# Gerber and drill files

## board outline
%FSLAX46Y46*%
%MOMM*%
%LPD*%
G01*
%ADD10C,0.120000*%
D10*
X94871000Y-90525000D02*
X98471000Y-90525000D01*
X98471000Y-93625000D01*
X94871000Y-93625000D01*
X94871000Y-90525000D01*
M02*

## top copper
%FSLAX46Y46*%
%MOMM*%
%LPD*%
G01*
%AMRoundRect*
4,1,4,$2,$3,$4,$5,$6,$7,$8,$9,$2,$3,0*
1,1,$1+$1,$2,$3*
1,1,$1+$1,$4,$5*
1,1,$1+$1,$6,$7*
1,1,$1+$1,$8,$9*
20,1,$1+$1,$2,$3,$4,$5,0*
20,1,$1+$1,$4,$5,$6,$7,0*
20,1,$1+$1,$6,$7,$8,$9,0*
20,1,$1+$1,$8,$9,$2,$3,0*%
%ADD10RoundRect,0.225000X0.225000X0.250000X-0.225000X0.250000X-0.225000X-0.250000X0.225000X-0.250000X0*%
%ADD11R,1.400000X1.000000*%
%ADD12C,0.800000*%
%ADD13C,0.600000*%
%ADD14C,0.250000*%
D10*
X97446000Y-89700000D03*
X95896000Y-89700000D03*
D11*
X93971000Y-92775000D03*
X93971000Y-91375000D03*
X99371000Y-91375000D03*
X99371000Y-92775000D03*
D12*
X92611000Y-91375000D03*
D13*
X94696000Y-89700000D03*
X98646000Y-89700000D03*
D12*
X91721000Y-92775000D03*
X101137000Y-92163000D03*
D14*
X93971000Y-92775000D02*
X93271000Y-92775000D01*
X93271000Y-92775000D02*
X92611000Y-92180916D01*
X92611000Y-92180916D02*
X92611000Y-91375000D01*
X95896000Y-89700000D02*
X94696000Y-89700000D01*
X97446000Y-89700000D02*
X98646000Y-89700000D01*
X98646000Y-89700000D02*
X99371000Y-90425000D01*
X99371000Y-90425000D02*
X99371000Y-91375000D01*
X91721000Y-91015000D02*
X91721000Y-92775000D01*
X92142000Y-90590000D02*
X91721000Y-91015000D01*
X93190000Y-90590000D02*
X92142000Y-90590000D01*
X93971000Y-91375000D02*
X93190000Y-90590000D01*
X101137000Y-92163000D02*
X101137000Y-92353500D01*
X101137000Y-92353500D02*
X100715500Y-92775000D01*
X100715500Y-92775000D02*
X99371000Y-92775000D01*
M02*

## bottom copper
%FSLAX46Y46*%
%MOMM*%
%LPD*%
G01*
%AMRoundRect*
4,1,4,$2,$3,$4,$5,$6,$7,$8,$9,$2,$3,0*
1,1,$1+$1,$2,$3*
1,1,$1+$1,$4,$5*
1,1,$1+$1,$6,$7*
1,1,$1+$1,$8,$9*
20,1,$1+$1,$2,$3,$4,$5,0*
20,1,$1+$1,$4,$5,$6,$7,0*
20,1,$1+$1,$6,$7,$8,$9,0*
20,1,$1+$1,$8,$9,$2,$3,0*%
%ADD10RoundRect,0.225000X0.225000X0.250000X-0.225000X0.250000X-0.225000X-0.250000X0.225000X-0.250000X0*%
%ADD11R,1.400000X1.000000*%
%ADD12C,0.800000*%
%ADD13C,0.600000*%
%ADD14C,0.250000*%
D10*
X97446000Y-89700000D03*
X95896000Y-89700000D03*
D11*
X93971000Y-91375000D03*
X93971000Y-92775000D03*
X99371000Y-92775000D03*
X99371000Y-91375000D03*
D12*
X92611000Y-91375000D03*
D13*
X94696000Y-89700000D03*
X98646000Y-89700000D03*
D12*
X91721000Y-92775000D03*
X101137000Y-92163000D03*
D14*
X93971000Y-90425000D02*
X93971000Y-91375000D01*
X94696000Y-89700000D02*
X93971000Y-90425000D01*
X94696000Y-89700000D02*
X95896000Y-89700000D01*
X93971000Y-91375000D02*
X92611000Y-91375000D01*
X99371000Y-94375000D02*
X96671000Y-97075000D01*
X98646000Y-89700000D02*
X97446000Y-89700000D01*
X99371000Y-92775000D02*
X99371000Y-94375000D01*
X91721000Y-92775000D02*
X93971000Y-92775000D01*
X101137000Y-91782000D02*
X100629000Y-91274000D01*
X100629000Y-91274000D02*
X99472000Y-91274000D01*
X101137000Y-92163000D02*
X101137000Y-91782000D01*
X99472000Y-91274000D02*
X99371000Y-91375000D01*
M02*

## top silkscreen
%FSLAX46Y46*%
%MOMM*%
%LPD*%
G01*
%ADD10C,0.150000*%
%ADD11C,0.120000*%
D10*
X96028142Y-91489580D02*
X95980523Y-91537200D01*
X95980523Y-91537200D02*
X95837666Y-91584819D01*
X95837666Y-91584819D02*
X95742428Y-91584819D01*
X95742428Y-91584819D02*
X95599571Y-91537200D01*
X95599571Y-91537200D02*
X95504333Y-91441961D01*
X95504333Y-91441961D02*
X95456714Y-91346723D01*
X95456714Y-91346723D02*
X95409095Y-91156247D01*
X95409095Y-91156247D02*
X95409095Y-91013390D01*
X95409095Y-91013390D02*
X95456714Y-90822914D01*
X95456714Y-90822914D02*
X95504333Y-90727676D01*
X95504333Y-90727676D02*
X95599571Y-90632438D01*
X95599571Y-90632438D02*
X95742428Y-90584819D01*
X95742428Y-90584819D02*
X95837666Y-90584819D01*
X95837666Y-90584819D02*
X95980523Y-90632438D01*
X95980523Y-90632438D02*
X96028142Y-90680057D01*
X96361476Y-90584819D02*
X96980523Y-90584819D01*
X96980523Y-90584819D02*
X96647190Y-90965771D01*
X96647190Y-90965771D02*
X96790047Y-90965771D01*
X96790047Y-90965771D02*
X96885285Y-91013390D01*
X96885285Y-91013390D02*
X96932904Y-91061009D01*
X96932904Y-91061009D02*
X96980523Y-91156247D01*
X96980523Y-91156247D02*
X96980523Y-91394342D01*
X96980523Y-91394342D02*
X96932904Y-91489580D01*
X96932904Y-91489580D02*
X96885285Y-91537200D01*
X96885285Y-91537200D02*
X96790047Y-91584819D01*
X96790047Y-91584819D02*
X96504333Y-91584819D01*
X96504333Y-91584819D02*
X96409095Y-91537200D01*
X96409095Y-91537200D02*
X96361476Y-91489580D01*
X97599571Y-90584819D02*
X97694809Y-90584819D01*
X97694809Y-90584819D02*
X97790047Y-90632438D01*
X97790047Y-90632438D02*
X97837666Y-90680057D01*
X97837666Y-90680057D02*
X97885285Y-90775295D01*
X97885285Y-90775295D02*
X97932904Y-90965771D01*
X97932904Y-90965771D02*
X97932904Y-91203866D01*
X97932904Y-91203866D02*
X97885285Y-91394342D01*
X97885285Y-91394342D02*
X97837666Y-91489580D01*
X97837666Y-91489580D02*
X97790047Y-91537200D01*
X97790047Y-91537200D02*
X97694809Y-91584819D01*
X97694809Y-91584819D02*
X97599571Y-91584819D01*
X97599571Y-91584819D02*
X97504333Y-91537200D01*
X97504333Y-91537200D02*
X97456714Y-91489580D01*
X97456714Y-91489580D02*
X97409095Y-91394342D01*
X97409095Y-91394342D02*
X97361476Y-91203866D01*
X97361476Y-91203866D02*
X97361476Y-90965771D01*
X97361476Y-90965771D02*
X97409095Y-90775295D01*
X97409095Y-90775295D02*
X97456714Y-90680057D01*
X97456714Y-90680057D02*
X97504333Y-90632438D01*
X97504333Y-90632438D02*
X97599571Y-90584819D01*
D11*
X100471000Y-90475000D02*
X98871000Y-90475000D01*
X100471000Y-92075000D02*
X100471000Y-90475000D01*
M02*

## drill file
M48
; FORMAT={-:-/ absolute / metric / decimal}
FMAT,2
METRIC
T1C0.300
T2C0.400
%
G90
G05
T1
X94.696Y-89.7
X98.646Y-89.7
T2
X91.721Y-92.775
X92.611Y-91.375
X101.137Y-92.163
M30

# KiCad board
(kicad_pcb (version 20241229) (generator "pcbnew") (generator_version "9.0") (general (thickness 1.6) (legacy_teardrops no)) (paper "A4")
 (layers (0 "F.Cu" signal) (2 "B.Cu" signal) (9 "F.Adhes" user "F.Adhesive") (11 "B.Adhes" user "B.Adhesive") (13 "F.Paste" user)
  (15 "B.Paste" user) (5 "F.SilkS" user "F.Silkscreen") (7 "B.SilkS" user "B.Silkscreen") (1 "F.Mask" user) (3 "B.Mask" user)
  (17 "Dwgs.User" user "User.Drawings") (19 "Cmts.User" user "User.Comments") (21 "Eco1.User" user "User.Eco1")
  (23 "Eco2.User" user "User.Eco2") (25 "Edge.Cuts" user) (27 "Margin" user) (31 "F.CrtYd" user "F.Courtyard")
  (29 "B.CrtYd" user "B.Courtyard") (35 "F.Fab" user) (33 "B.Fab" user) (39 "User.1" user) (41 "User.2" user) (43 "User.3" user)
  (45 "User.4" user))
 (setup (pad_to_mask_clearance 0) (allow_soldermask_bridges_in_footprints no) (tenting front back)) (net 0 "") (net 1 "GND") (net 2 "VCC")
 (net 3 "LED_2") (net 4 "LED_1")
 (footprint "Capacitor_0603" (layer "F.Cu") (at 96.671 89.7 180)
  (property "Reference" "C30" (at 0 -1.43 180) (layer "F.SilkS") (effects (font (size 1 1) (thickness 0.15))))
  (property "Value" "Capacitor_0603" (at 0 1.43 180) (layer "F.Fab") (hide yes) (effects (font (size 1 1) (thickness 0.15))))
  (pad "1" smd roundrect (at -0.775 0 180) (size 0.9 0.95) (layers "F.Cu" "F.Mask" "F.Paste") (roundrect_rratio 0.25) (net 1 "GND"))
  (pad "1" smd roundrect (at -0.775 0 180) (size 0.9 0.95) (layers "B.Cu" "B.Mask" "B.Paste") (roundrect_rratio 0.25) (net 1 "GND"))
  (pad "2" smd roundrect (at 0.775 0 180) (size 0.9 0.95) (layers "F.Cu" "F.Mask" "F.Paste") (roundrect_rratio 0.25) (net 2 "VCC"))
  (pad "2" smd roundrect (at 0.775 0 180) (size 0.9 0.95) (layers "B.Cu" "B.Mask" "B.Paste") (roundrect_rratio 0.25) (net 2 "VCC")))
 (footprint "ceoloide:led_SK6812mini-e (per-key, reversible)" (layer "B.Cu") (at 96.671 92.075 180)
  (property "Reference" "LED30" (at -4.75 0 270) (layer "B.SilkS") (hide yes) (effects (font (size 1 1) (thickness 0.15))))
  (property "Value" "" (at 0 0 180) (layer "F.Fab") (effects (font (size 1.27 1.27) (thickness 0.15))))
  (fp_line (start -3.8 1.6) (end -2.2 1.6) (stroke (width 0.12) (type solid)) (layer "F.SilkS"))
  (fp_line (start -3.8 0) (end -3.8 1.6) (stroke (width 0.12) (type solid)) (layer "F.SilkS"))
  (fp_rect (start -1.8 -1.55) (end 1.8 1.55) (stroke (width 0.12) (type solid)) (fill no) (layer "Edge.Cuts"))
  (pad "1" smd rect (at 2.7 -0.7 180) (size 1.4 1) (layers "F.Cu" "F.Mask" "F.Paste") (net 2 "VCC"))
  (pad "1" smd rect (at 2.7 0.7 180) (size 1.4 1) (layers "B.Cu" "B.Mask" "B.Paste") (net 2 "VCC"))
  (pad "2" smd rect (at 2.7 -0.7 180) (size 1.4 1) (layers "B.Cu" "B.Mask" "B.Paste") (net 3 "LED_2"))
  (pad "2" smd rect (at 2.7 0.7 180) (size 1.4 1) (layers "F.Cu" "F.Mask" "F.Paste") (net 3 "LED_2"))
  (pad "3" smd rect (at -2.7 -0.7 180) (size 1.4 1) (layers "B.Cu" "B.Mask" "B.Paste") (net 1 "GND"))
  (pad "3" smd rect (at -2.7 0.7 180) (size 1.4 1) (layers "F.Cu" "F.Mask" "F.Paste") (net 1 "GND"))
  (pad "4" smd rect (at -2.7 -0.7 180) (size 1.4 1) (layers "F.Cu" "F.Mask" "F.Paste") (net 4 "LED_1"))
  (pad "4" smd rect (at -2.7 0.7 180) (size 1.4 1) (layers "B.Cu" "B.Mask" "B.Paste") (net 4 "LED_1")))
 (segment (start 93.971 92.775) (end 93.271 92.775) (width 0.25) (layer "F.Cu") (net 2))
 (segment (start 93.271 92.775) (end 92.611 92.180916) (width 0.25) (layer "F.Cu") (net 2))
 (segment (start 92.611 92.180916) (end 92.611 91.375) (width 0.25) (layer "F.Cu") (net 2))
 (segment (start 95.896 89.7) (end 94.696 89.7) (width 0.25) (layer "F.Cu") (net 2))
 (via (at 92.611 91.375) (size 0.8) (drill 0.4) (layers "F.Cu" "B.Cu") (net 2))
 (via (at 94.696 89.7) (size 0.6) (drill 0.3) (layers "F.Cu" "B.Cu") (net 2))
 (segment (start 93.971 90.425) (end 93.971 91.375) (width 0.25) (layer "B.Cu") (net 2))
 (segment (start 94.696 89.7) (end 93.971 90.425) (width 0.25) (layer "B.Cu") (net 2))
 (segment (start 94.696 89.7) (end 95.896 89.7) (width 0.25) (layer "B.Cu") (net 2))
 (segment (start 93.971 91.375) (end 92.611 91.375) (width 0.25) (layer "B.Cu") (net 2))
 (segment (start 97.446 89.7) (end 98.646 89.7) (width 0.25) (layer "F.Cu") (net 1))
 (segment (start 98.646 89.7) (end 99.371 90.425) (width 0.25) (layer "F.Cu") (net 1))
 (segment (start 99.371 90.425) (end 99.371 91.375) (width 0.25) (layer "F.Cu") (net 1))
 (via (at 98.646 89.7) (size 0.6) (drill 0.3) (layers "F.Cu" "B.Cu") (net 1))
 (segment (start 99.371 94.375) (end 96.671 97.075) (width 0.25) (layer "B.Cu") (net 1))
 (segment (start 98.646 89.7) (end 97.446 89.7) (width 0.25) (layer "B.Cu") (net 1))
 (segment (start 99.371 92.775) (end 99.371 94.375) (width 0.25) (layer "B.Cu") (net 1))
 (segment (start 91.721 91.015) (end 91.721 92.775) (width 0.25) (layer "F.Cu") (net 3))
 (segment (start 92.142 90.59) (end 91.721 91.015) (width 0.25) (layer "F.Cu") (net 3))
 (segment (start 93.19 90.59) (end 92.142 90.59) (width 0.25) (layer "F.Cu") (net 3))
 (segment (start 93.971 91.375) (end 93.19 90.59) (width 0.25) (layer "F.Cu") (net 3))
 (via (at 91.721 92.775) (size 0.8) (drill 0.4) (layers "F.Cu" "B.Cu") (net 3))
 (segment (start 91.721 92.775) (end 93.971 92.775) (width 0.25) (layer "B.Cu") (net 3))
 (segment (start 101.137 92.163) (end 101.137 92.3535) (width 0.25) (layer "F.Cu") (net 4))
 (segment (start 101.137 92.3535) (end 100.7155 92.775) (width 0.25) (layer "F.Cu") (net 4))
 (segment (start 100.7155 92.775) (end 99.371 92.775) (width 0.25) (layer "F.Cu") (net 4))
 (via (at 101.137 92.163) (size 0.8) (drill 0.4) (layers "F.Cu" "B.Cu") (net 4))
 (segment (start 101.137 91.782) (end 100.629 91.274) (width 0.25) (layer "B.Cu") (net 4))
 (segment (start 100.629 91.274) (end 99.472 91.274) (width 0.25) (layer "B.Cu") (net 4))
 (segment (start 101.137 92.163) (end 101.137 91.782) (width 0.25) (layer "B.Cu") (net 4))
 (segment (start 99.472 91.274) (end 99.371 91.375) (width 0.25) (layer "B.Cu") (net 4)))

